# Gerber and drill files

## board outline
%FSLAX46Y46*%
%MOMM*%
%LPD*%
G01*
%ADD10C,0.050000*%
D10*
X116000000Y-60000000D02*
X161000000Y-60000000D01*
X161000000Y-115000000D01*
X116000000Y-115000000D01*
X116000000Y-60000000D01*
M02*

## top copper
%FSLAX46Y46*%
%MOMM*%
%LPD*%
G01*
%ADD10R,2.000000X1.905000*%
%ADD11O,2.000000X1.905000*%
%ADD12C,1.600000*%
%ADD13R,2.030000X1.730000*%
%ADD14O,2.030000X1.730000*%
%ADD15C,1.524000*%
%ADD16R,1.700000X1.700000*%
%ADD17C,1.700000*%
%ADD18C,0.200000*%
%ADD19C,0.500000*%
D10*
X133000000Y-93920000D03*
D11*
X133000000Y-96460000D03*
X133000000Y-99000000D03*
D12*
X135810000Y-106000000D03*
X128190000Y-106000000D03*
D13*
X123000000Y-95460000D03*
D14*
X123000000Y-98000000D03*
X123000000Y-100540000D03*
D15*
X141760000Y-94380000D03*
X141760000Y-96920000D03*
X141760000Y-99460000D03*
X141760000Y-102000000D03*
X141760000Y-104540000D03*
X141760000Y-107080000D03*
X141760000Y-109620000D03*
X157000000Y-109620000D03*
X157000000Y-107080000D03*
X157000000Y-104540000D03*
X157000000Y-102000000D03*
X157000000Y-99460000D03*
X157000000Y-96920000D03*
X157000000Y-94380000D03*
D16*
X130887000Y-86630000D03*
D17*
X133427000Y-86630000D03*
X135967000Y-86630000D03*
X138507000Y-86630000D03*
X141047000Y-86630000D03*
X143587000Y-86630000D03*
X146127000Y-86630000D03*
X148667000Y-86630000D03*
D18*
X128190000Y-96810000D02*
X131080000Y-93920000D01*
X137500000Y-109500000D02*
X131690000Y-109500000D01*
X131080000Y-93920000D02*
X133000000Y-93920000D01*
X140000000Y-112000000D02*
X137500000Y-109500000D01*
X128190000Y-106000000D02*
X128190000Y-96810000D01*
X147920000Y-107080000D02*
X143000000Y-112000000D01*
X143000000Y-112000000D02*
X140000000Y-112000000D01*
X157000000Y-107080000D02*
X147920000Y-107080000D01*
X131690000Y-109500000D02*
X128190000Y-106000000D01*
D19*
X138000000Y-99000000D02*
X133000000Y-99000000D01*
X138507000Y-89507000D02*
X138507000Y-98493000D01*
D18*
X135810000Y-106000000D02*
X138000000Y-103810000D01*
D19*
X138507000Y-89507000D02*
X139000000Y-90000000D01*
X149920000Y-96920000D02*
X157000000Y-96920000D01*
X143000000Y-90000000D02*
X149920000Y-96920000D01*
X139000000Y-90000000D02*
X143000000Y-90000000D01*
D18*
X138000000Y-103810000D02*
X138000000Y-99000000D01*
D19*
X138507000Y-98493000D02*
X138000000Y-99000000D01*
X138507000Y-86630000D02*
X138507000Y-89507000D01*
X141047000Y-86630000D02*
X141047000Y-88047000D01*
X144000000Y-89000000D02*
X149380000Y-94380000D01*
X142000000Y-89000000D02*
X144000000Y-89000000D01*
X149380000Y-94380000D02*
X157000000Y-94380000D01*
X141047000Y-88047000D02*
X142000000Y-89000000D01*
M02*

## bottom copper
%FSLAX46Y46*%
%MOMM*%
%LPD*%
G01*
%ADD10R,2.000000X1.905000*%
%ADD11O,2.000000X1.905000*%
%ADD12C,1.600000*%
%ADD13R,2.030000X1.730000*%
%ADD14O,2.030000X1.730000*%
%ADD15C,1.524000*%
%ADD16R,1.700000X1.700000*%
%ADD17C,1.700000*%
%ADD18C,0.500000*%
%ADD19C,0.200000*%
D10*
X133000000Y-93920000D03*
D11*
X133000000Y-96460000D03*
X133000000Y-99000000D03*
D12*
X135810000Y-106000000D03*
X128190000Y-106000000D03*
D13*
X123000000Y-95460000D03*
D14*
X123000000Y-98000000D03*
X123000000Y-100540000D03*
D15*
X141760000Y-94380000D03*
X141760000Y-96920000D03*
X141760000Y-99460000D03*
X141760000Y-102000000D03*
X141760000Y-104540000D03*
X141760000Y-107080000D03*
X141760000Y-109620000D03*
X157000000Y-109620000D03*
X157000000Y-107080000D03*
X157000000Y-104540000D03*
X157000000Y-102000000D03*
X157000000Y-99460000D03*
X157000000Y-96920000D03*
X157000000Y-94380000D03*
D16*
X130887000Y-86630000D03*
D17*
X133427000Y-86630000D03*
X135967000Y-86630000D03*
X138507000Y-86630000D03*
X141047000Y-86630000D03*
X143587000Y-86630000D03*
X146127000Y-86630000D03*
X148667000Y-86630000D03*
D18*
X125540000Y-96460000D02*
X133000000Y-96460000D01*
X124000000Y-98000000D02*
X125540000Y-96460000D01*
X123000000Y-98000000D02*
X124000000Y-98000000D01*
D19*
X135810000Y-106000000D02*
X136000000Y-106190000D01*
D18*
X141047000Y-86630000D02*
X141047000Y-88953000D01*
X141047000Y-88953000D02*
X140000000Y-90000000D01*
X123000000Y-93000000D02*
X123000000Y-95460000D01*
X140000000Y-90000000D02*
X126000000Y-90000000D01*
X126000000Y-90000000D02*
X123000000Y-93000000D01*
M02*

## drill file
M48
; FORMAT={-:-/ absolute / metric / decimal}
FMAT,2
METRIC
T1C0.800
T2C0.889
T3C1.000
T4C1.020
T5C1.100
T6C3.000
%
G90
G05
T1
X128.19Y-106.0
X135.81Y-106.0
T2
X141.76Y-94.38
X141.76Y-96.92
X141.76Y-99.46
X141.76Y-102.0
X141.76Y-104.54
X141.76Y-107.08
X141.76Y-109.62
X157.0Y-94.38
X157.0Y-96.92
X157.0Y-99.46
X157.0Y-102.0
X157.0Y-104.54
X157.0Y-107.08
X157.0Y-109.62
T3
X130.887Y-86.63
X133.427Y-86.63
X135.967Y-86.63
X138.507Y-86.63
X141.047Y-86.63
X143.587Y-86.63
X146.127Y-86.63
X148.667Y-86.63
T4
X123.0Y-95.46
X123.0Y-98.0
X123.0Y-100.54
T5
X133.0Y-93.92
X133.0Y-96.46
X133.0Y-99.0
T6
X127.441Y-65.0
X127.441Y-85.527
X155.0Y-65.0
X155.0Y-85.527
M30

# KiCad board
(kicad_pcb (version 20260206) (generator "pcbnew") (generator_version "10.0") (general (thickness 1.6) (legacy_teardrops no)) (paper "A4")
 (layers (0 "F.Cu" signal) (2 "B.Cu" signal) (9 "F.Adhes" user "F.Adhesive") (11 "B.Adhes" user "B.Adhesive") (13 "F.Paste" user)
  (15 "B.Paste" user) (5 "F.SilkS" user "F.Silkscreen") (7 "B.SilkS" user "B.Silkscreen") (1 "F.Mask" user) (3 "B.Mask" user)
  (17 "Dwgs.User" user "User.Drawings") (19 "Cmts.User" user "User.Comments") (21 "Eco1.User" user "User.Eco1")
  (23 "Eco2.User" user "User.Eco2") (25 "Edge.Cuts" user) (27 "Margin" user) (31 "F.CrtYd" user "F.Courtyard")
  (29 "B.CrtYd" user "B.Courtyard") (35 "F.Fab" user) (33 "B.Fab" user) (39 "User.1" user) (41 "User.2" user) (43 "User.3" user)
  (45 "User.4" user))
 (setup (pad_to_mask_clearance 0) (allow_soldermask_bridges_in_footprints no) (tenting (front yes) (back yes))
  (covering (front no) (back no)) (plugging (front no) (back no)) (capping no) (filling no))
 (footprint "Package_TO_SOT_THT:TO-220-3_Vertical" (layer "F.Cu") (at 133 93.92 -90)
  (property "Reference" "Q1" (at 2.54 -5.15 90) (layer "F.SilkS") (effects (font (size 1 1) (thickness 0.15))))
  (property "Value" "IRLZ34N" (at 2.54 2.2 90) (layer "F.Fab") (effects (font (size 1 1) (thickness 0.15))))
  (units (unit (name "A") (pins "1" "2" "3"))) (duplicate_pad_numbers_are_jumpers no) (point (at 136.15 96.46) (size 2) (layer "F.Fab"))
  (pad "1" thru_hole rect (at 0 0 270) (size 1.905 2) (drill 1.1) (layers "*.Cu" "*.Mask") (remove_unused_layers no) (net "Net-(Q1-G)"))
  (pad "2" thru_hole oval (at 2.54 0 270) (size 1.905 2) (drill 1.1) (layers "*.Cu" "*.Mask") (remove_unused_layers no)
   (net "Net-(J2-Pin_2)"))
  (pad "3" thru_hole oval (at 5.08 0 270) (size 1.905 2) (drill 1.1) (layers "*.Cu" "*.Mask") (remove_unused_layers no) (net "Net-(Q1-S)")))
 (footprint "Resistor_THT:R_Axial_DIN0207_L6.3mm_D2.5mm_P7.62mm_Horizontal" (layer "F.Cu") (at 135.81 106 180)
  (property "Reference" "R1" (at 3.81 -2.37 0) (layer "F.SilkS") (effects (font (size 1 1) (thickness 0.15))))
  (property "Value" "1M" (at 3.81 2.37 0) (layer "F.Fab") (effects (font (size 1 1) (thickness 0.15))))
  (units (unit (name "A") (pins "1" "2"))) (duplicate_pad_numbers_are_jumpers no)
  (pad "1" thru_hole circle (at 0 0 180) (size 1.6 1.6) (drill 0.8) (layers "*.Cu" "*.Mask") (remove_unused_layers no) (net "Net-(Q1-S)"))
  (pad "2" thru_hole circle (at 7.62 0 180) (size 1.6 1.6) (drill 0.8) (layers "*.Cu" "*.Mask") (remove_unused_layers no) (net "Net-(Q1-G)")))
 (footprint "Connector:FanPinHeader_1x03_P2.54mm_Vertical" (layer "F.Cu") (at 123 95.46 -90)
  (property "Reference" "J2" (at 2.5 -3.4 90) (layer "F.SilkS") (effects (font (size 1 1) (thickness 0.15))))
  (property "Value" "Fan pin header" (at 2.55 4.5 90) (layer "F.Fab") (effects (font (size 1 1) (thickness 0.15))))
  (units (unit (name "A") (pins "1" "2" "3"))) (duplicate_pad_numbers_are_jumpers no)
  (pad "1" thru_hole rect (at 0 0) (size 2.03 1.73) (drill 1.02) (layers "*.Cu" "*.Mask") (remove_unused_layers no) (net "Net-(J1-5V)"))
  (pad "2" thru_hole oval (at 2.54 0) (size 2.03 1.73) (drill 1.02) (layers "*.Cu" "*.Mask") (remove_unused_layers no)
   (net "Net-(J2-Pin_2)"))
  (pad "3" thru_hole oval (at 5.08 0) (size 2.03 1.73) (drill 1.02) (layers "*.Cu" "*.Mask") (remove_unused_layers no)
   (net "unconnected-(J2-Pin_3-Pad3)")))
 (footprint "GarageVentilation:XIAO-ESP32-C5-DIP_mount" (layer "F.Cu") (at 149.38 102 90)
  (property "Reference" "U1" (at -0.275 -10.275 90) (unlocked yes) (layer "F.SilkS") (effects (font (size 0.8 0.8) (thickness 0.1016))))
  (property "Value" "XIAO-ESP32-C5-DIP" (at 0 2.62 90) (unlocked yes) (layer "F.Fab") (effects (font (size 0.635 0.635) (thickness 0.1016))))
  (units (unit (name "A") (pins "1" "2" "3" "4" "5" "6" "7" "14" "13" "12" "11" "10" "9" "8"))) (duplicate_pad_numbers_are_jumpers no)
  (pad "1" thru_hole circle (at 7.62 -7.62 180) (size 1.524 1.524) (drill 0.889) (layers "*.Cu" "*.Mask") (remove_unused_layers no)
   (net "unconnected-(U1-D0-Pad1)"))
  (pad "2" thru_hole circle (at 5.08 -7.62 180) (size 1.524 1.524) (drill 0.889) (layers "*.Cu" "*.Mask") (remove_unused_layers no)
   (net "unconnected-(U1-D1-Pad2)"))
  (pad "3" thru_hole circle (at 2.54 -7.62 180) (size 1.524 1.524) (drill 0.889) (layers "*.Cu" "*.Mask") (remove_unused_layers no)
   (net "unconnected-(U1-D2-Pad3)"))
  (pad "4" thru_hole circle (at 0 -7.62 180) (size 1.524 1.524) (drill 0.889) (layers "*.Cu" "*.Mask") (remove_unused_layers no)
   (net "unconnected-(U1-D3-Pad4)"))
  (pad "5" thru_hole circle (at -2.54 -7.62 180) (size 1.524 1.524) (drill 0.889) (layers "*.Cu" "*.Mask") (remove_unused_layers no)
   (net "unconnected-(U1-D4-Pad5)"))
  (pad "6" thru_hole circle (at -5.08 -7.62 180) (size 1.524 1.524) (drill 0.889) (layers "*.Cu" "*.Mask") (remove_unused_layers no)
   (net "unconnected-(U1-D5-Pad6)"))
  (pad "7" thru_hole circle (at -7.62 -7.62 180) (size 1.524 1.524) (drill 0.889) (layers "*.Cu" "*.Mask") (remove_unused_layers no)
   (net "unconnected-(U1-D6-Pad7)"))
  (pad "8" thru_hole circle (at -7.62 7.62) (size 1.524 1.524) (drill 0.889) (layers "*.Cu" "*.Mask") (remove_unused_layers no)
   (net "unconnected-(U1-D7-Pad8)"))
  (pad "9" thru_hole circle (at -5.08 7.62) (size 1.524 1.524) (drill 0.889) (layers "*.Cu" "*.Mask") (remove_unused_layers no)
   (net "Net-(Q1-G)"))
  (pad "10" thru_hole circle (at -2.54 7.62) (size 1.524 1.524) (drill 0.889) (layers "*.Cu" "*.Mask") (remove_unused_layers no)
   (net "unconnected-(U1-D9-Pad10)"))
  (pad "11" thru_hole circle (at 0 7.62) (size 1.524 1.524) (drill 0.889) (layers "*.Cu" "*.Mask") (remove_unused_layers no)
   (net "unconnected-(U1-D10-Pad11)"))
  (pad "12" thru_hole circle (at 2.54 7.62) (size 1.524 1.524) (drill 0.889) (layers "*.Cu" "*.Mask") (remove_unused_layers no)
   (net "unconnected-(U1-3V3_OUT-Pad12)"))
  (pad "13" thru_hole circle (at 5.08 7.62) (size 1.524 1.524) (drill 0.889) (layers "*.Cu" "*.Mask") (remove_unused_layers no)
   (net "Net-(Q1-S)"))
  (pad "14" thru_hole circle (at 7.62 7.62) (size 1.524 1.524) (drill 0.889) (layers "*.Cu" "*.Mask") (remove_unused_layers no)
   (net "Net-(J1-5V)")))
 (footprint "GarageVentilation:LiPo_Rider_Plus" (layer "F.Cu") (at 130.887 86.63)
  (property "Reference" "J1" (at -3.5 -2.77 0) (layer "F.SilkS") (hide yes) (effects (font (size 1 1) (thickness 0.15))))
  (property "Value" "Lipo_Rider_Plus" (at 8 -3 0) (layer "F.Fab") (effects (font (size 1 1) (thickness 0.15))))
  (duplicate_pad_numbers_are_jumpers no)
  (pad "" np_thru_hole circle (at -3.446 -21.63) (size 3 3) (drill 3) (layers "*.Cu" "*.Mask"))
  (pad "" np_thru_hole circle (at -3.446 -1.103) (size 3 3) (drill 3) (layers "*.Cu" "*.Mask"))
  (pad "" np_thru_hole circle (at 24.113 -21.63) (size 3 3) (drill 3) (layers "*.Cu" "*.Mask"))
  (pad "" np_thru_hole circle (at 24.113 -1.103) (size 3 3) (drill 3) (layers "*.Cu" "*.Mask"))
  (pad "1" thru_hole rect (at 0 0) (size 1.7 1.7) (drill 1) (layers "*.Cu" "*.Mask") (remove_unused_layers no)
   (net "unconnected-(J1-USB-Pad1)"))
  (pad "2" thru_hole circle (at 2.54 0) (size 1.7 1.7) (drill 1) (layers "*.Cu" "*.Mask") (remove_unused_layers no)
   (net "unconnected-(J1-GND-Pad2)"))
  (pad "3" thru_hole circle (at 5.08 0) (size 1.7 1.7) (drill 1) (layers "*.Cu" "*.Mask") (remove_unused_layers no)
   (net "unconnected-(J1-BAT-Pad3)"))
  (pad "4" thru_hole circle (at 7.62 0) (size 1.7 1.7) (drill 1) (layers "*.Cu" "*.Mask") (remove_unused_layers no) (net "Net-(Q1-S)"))
  (pad "5" thru_hole circle (at 10.16 0) (size 1.7 1.7) (drill 1) (layers "*.Cu" "*.Mask") (remove_unused_layers no) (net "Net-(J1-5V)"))
  (pad "6" thru_hole circle (at 12.7 0) (size 1.7 1.7) (drill 1) (layers "*.Cu" "*.Mask") (remove_unused_layers no)
   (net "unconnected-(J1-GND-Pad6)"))
  (pad "7" thru_hole circle (at 15.24 0) (size 1.7 1.7) (drill 1) (layers "*.Cu" "*.Mask") (remove_unused_layers no)
   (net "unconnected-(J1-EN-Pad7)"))
  (pad "8" thru_hole circle (at 17.78 0) (size 1.7 1.7) (drill 1) (layers "*.Cu" "*.Mask") (remove_unused_layers no)
   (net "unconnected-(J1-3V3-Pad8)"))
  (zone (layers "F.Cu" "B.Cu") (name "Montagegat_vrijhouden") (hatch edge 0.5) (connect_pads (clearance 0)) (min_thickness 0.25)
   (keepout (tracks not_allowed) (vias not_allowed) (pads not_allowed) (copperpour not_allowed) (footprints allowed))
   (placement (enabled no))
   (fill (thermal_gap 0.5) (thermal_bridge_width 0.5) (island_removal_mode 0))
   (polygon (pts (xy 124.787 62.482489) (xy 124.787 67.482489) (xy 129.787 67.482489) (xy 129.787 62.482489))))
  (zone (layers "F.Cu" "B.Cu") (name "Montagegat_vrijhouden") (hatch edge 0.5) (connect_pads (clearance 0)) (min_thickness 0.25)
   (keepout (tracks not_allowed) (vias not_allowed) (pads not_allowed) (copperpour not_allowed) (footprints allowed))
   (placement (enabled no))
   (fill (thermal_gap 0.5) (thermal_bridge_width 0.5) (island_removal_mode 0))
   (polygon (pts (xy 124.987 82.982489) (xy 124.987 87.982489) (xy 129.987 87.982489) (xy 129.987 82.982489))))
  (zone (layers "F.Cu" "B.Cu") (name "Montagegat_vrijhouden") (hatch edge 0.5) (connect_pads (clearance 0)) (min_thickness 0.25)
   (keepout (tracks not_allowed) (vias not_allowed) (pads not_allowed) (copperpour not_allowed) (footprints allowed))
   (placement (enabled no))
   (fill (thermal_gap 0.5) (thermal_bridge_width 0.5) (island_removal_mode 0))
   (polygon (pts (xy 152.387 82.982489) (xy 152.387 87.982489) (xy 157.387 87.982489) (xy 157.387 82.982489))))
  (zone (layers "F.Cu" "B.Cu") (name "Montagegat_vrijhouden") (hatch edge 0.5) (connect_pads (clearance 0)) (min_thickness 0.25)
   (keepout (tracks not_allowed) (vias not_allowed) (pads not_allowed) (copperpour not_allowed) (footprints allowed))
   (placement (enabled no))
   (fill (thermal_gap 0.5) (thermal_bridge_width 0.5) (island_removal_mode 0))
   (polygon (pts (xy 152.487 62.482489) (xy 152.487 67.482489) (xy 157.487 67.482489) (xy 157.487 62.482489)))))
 (gr_rect (start 116 60) (end 161 115) (stroke (width 0.05) (type default)) (fill no) (layer "Edge.Cuts"))
 (segment (start 128.19 96.81) (end 131.08 93.92) (width 0.2) (layer "F.Cu") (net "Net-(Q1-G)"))
 (segment (start 137.5 109.5) (end 131.69 109.5) (width 0.2) (layer "F.Cu") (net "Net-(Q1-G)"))
 (segment (start 131.08 93.92) (end 133 93.92) (width 0.2) (layer "F.Cu") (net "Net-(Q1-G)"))
 (segment (start 140 112) (end 137.5 109.5) (width 0.2) (layer "F.Cu") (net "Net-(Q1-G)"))
 (segment (start 128.19 106) (end 128.19 96.81) (width 0.2) (layer "F.Cu") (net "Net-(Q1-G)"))
 (segment (start 147.92 107.08) (end 143 112) (width 0.2) (layer "F.Cu") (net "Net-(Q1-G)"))
 (segment (start 143 112) (end 140 112) (width 0.2) (layer "F.Cu") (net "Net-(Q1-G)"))
 (segment (start 157 107.08) (end 147.92 107.08) (width 0.2) (layer "F.Cu") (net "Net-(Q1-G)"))
 (segment (start 131.69 109.5) (end 128.19 106) (width 0.2) (layer "F.Cu") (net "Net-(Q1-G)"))
 (segment (start 125.54 96.46) (end 133 96.46) (width 0.5) (layer "B.Cu") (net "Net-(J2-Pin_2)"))
 (segment (start 124 98) (end 125.54 96.46) (width 0.5) (layer "B.Cu") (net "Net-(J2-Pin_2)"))
 (segment (start 123 98) (end 124 98) (width 0.5) (layer "B.Cu") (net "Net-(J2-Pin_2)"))
 (segment (start 138 99) (end 133 99) (width 0.5) (layer "F.Cu") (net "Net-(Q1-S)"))
 (segment (start 138.507 89.507) (end 138.507 98.493) (width 0.5) (layer "F.Cu") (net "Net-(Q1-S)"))
 (segment (start 135.81 106) (end 138 103.81) (width 0.2) (layer "F.Cu") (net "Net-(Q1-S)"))
 (segment (start 138.507 89.507) (end 139 90) (width 0.5) (layer "F.Cu") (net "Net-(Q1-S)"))
 (segment (start 149.92 96.92) (end 157 96.92) (width 0.5) (layer "F.Cu") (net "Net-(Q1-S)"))
 (segment (start 143 90) (end 149.92 96.92) (width 0.5) (layer "F.Cu") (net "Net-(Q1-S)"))
 (segment (start 139 90) (end 143 90) (width 0.5) (layer "F.Cu") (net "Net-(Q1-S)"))
 (segment (start 138 103.81) (end 138 99) (width 0.2) (layer "F.Cu") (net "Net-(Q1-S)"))
 (segment (start 138.507 98.493) (end 138 99) (width 0.5) (layer "F.Cu") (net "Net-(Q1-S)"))
 (segment (start 138.507 86.63) (end 138.507 89.507) (width 0.5) (layer "F.Cu") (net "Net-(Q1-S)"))
 (segment (start 135.81 106) (end 136 106.19) (width 0.2) (layer "B.Cu") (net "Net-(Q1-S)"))
 (segment (start 141.047 86.63) (end 141.047 88.047) (width 0.5) (layer "F.Cu") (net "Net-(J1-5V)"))
 (segment (start 144 89) (end 149.38 94.38) (width 0.5) (layer "F.Cu") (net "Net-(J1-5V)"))
 (segment (start 142 89) (end 144 89) (width 0.5) (layer "F.Cu") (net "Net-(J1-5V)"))
 (segment (start 149.38 94.38) (end 157 94.38) (width 0.5) (layer "F.Cu") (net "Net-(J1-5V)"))
 (segment (start 141.047 88.047) (end 142 89) (width 0.5) (layer "F.Cu") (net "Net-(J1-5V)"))
 (segment (start 141.047 86.63) (end 141.047 88.953) (width 0.5) (layer "B.Cu") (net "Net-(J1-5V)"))
 (segment (start 141.047 88.953) (end 140 90) (width 0.5) (layer "B.Cu") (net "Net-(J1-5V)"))
 (segment (start 123 93) (end 123 95.46) (width 0.5) (layer "B.Cu") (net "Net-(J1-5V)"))
 (segment (start 140 90) (end 126 90) (width 0.5) (layer "B.Cu") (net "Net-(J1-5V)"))
 (segment (start 126 90) (end 123 93) (width 0.5) (layer "B.Cu") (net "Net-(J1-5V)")))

